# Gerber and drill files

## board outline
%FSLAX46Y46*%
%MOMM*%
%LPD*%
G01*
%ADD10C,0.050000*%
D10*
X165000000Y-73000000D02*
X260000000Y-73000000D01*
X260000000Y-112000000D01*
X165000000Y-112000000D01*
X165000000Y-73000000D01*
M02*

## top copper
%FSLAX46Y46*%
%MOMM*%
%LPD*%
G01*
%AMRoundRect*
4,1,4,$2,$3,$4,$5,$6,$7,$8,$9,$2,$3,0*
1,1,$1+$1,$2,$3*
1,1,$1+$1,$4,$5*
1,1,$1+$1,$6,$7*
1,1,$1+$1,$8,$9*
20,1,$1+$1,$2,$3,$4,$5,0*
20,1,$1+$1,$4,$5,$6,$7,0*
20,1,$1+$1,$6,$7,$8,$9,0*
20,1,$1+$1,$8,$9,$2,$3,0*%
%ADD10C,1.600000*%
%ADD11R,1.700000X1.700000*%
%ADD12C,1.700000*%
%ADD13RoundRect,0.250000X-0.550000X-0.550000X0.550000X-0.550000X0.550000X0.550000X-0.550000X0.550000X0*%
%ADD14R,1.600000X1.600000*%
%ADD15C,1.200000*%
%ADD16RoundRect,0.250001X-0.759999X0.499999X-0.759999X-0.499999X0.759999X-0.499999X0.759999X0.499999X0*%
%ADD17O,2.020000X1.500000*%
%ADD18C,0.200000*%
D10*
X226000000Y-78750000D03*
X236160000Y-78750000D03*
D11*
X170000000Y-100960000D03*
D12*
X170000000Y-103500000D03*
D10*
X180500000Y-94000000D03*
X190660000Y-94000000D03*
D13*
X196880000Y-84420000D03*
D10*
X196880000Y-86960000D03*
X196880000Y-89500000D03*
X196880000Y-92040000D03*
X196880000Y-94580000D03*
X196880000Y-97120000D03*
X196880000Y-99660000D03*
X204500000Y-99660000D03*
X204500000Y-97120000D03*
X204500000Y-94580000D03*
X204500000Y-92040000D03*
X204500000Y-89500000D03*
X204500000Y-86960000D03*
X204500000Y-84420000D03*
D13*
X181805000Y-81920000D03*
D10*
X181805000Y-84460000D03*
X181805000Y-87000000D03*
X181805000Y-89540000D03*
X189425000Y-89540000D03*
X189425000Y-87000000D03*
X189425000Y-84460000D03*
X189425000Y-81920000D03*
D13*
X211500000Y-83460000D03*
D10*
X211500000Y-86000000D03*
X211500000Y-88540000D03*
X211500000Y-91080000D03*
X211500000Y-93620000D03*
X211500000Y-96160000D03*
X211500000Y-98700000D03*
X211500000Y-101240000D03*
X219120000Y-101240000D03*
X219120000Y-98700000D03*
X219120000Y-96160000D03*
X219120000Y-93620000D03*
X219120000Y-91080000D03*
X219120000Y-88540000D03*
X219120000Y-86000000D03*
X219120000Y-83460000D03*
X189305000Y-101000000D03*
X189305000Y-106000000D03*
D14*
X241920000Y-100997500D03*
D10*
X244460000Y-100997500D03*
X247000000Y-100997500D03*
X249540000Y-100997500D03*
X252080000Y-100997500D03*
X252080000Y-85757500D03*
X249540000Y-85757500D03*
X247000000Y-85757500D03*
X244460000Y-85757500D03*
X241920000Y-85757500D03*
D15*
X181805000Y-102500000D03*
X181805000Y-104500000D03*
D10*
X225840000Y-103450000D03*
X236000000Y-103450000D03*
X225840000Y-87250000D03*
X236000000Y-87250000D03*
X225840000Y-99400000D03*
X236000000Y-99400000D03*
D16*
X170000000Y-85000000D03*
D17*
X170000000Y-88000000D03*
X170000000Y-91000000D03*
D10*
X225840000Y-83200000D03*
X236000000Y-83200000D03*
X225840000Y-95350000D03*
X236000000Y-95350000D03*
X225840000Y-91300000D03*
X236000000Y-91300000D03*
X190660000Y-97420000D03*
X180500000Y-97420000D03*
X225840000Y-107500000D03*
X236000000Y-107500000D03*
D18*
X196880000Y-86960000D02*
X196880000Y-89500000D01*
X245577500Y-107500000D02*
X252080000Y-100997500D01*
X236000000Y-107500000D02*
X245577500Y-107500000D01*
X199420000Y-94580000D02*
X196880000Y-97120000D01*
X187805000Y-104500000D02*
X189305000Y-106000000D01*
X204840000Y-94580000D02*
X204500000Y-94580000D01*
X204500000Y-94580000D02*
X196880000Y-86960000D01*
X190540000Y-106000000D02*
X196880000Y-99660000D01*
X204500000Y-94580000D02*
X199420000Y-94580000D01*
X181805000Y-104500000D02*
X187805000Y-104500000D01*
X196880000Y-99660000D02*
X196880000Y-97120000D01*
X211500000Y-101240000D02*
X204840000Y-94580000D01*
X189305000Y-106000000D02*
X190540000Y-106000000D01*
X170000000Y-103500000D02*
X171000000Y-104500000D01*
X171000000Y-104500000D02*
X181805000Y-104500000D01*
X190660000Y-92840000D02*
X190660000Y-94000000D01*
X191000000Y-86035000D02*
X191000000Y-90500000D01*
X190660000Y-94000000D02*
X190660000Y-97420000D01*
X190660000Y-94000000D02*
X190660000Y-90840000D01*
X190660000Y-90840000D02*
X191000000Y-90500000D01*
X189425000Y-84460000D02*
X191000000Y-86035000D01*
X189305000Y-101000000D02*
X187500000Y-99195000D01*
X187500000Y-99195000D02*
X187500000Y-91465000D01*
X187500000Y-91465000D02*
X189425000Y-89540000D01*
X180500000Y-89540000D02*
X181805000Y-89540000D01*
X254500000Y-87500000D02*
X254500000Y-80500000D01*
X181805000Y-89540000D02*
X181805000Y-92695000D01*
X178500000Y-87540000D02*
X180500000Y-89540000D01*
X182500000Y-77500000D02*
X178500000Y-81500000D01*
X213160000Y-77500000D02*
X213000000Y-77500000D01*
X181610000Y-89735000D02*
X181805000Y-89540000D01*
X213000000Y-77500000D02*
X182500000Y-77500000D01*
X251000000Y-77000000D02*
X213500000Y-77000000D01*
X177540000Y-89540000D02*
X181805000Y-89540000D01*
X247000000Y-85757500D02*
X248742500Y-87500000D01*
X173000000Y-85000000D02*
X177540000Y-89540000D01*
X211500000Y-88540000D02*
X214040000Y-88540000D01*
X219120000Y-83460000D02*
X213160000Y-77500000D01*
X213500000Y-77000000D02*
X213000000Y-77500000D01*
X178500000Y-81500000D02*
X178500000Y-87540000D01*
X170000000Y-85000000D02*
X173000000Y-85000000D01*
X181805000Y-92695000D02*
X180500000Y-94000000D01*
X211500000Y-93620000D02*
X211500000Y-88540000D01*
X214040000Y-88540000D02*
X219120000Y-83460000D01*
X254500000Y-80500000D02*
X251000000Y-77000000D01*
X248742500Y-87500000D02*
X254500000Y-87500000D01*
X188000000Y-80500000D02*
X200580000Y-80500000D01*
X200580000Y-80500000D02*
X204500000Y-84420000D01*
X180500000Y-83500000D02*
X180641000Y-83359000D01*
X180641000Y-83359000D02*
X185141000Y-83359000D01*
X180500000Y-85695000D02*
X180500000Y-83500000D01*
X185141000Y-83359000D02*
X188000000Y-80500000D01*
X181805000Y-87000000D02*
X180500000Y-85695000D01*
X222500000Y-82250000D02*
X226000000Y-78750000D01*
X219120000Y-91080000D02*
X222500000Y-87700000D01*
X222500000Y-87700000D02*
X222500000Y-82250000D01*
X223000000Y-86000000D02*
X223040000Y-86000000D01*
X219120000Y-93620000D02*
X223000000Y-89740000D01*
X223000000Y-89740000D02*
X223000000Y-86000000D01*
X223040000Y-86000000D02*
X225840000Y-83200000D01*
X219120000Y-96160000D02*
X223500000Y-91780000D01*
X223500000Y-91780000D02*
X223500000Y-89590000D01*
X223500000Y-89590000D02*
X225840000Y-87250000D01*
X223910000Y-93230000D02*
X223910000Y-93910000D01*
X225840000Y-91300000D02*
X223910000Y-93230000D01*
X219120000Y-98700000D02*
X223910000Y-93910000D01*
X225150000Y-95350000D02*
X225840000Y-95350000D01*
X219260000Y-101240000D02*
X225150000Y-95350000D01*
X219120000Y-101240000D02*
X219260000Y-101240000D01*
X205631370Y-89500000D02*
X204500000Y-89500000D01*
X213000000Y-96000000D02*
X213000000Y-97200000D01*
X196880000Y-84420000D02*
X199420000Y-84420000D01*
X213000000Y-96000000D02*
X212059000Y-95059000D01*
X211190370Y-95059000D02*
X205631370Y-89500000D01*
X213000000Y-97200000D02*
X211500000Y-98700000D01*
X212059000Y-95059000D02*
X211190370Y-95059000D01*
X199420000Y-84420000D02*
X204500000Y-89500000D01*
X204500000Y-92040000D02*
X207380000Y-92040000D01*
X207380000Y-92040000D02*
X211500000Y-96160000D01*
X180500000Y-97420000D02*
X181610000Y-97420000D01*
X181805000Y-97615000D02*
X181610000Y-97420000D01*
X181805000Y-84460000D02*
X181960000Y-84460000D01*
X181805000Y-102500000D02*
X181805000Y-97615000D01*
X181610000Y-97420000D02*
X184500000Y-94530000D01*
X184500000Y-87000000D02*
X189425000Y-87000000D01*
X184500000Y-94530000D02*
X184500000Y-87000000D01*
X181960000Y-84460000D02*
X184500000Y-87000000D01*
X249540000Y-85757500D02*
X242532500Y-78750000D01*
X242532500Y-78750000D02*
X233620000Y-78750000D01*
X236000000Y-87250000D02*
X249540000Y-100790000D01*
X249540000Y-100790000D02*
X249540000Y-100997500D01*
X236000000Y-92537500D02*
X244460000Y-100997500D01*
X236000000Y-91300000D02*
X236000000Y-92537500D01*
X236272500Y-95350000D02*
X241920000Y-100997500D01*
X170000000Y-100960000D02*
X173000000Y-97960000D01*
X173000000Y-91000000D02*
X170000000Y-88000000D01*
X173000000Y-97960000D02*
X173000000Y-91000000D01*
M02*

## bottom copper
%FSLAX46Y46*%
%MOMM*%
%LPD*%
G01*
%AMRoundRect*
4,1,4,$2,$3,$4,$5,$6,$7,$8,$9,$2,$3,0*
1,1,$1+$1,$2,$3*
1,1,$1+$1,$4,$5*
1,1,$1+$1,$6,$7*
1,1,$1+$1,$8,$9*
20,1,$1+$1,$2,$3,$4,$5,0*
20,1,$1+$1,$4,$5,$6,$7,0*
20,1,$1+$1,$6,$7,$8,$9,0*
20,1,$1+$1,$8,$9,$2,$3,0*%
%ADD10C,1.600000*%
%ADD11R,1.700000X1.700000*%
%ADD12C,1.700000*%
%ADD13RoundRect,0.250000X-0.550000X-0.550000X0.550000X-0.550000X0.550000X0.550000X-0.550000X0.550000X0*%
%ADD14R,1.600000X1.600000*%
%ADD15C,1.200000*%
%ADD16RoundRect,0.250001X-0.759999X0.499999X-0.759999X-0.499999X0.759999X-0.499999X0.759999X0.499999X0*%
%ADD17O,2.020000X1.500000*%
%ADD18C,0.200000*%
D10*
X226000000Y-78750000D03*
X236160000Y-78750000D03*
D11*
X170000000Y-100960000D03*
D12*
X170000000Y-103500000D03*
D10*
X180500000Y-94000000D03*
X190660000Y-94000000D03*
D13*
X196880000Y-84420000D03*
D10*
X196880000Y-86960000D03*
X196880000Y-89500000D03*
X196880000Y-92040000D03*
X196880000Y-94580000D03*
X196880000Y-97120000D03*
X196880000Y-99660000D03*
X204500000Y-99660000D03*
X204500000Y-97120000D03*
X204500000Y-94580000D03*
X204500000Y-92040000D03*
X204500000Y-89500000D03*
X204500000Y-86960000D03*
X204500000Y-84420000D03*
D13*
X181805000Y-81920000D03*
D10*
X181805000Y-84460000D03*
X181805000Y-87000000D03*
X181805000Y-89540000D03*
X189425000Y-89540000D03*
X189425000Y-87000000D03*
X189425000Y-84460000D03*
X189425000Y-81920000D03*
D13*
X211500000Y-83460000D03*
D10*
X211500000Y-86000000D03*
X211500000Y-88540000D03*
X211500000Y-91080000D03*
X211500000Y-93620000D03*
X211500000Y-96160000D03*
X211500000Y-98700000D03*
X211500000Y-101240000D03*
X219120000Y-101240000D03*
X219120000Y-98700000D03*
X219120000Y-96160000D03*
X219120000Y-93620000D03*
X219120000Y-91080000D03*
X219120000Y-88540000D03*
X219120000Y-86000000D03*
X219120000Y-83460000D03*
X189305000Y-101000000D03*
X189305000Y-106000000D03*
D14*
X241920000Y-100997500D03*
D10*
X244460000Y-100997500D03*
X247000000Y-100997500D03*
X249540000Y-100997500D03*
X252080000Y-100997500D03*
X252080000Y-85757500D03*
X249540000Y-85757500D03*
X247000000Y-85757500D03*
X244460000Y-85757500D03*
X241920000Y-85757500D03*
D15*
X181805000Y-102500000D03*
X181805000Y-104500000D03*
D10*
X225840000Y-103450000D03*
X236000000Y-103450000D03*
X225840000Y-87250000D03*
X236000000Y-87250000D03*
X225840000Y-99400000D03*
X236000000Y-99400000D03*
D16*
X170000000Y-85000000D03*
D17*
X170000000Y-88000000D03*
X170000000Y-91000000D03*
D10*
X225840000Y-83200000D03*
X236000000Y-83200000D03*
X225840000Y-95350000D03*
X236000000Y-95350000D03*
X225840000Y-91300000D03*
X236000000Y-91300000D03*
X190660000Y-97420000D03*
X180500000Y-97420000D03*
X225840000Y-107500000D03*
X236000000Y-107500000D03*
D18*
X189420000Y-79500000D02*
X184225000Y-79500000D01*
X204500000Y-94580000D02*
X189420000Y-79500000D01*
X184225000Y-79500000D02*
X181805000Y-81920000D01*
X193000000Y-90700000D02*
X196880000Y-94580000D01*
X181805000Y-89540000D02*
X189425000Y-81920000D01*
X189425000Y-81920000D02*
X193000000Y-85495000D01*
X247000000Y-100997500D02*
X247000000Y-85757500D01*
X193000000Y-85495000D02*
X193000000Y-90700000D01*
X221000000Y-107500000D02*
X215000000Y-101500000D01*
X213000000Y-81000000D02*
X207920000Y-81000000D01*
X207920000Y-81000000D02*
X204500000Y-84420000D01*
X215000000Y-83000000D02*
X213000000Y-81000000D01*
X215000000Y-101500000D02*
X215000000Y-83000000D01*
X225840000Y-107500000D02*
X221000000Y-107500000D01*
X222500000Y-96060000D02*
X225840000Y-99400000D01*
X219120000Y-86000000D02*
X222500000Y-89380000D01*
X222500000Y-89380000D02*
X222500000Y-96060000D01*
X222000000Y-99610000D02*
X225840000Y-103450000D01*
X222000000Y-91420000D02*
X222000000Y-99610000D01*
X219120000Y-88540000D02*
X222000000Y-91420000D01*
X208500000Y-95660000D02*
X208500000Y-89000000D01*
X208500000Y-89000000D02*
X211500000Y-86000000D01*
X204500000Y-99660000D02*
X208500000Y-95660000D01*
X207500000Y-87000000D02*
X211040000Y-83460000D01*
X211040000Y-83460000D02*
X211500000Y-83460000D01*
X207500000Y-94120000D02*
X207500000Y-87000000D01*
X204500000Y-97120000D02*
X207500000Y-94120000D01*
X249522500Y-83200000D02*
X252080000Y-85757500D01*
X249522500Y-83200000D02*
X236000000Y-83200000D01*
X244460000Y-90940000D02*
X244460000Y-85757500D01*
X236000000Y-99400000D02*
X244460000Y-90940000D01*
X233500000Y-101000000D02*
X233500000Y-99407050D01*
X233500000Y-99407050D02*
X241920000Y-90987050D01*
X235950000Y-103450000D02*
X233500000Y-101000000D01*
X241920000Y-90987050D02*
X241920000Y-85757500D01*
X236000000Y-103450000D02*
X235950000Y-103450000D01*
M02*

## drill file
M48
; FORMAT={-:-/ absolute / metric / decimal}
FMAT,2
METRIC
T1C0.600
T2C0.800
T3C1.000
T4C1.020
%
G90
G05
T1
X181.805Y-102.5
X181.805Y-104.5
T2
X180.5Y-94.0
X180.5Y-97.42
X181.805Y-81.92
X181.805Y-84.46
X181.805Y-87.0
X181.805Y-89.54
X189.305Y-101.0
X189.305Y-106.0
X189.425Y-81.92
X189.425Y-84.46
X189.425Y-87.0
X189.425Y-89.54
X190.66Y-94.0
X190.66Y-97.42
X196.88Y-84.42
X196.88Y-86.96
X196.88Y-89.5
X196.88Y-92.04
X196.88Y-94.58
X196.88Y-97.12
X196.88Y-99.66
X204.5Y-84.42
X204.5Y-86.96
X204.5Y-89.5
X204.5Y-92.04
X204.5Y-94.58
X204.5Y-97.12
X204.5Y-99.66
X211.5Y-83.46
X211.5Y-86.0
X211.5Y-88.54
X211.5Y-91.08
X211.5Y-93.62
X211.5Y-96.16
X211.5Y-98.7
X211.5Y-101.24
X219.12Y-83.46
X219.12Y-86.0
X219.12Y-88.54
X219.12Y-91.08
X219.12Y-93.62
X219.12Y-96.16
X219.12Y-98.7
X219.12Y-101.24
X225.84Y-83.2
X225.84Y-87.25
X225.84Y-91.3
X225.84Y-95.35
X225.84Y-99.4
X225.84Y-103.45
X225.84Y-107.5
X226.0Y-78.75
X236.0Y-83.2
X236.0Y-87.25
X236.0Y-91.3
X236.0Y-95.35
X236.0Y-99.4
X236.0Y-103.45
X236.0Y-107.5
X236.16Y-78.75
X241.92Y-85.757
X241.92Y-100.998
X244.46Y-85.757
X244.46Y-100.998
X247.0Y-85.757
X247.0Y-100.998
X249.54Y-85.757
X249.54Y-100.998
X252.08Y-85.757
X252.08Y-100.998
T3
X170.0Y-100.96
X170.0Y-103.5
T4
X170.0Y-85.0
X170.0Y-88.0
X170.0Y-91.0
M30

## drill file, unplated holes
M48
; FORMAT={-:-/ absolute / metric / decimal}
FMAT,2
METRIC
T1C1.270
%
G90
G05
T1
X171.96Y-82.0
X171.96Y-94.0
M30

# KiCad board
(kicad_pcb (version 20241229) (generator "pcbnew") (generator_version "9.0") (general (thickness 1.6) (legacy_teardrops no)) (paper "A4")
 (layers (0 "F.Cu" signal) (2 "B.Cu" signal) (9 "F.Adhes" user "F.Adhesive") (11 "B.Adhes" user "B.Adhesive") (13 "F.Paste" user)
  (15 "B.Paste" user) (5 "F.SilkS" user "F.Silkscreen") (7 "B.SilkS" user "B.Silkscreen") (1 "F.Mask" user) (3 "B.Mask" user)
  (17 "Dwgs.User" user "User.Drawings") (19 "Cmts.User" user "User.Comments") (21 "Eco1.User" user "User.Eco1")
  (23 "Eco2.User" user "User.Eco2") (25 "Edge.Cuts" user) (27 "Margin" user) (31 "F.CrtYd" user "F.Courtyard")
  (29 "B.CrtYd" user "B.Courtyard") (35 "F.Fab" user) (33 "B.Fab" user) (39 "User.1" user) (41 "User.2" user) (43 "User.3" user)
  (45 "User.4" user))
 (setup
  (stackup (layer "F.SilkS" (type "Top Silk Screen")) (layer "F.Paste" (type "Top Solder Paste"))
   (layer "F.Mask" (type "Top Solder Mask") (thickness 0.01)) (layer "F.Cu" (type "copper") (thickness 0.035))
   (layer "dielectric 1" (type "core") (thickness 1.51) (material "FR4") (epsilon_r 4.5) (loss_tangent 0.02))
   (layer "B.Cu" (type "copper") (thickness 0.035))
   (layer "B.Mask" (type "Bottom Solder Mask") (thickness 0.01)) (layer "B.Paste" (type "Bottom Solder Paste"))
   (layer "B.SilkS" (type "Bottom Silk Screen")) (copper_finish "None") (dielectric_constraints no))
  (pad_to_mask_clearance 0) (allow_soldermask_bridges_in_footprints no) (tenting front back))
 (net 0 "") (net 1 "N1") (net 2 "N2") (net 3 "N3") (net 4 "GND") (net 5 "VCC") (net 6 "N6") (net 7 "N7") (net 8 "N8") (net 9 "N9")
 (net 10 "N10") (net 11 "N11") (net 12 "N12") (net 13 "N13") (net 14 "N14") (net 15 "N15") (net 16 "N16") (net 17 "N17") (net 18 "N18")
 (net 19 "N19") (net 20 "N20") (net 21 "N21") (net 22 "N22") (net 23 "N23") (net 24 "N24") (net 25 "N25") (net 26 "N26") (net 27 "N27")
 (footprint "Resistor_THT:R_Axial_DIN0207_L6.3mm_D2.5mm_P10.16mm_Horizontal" (layer "F.Cu") (at 226 78.75)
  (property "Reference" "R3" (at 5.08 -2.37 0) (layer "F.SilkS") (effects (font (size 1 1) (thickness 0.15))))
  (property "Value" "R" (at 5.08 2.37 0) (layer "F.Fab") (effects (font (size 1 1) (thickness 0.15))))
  (pad "1" thru_hole circle (at 0 0) (size 1.6 1.6) (drill 0.8) (layers "*.Cu" "*.Mask") (remove_unused_layers no) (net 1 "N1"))
  (pad "2" thru_hole circle (at 10.16 0) (size 1.6 1.6) (drill 0.8) (layers "*.Cu" "*.Mask") (remove_unused_layers no) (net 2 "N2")))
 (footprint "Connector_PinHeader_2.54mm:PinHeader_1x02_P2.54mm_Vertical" (layer "F.Cu") (at 170 100.96)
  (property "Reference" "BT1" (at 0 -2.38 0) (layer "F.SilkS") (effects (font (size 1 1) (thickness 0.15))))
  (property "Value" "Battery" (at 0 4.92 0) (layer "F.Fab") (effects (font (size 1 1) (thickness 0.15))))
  (pad "1" thru_hole rect (at 0 0) (size 1.7 1.7) (drill 1) (layers "*.Cu" "*.Mask") (remove_unused_layers no) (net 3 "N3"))
  (pad "2" thru_hole circle (at 0 2.54) (size 1.7 1.7) (drill 1) (layers "*.Cu" "*.Mask") (remove_unused_layers no) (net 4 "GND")))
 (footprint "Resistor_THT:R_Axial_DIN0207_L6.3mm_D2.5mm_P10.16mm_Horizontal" (layer "F.Cu") (at 180.5 94)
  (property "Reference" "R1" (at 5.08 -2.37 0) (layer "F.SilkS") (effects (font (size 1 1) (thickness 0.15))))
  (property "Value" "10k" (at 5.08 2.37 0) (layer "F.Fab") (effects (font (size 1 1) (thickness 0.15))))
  (pad "1" thru_hole circle (at 0 0) (size 1.6 1.6) (drill 0.8) (layers "*.Cu" "*.Mask") (remove_unused_layers no) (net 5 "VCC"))
  (pad "2" thru_hole circle (at 10.16 0) (size 1.6 1.6) (drill 0.8) (layers "*.Cu" "*.Mask") (remove_unused_layers no) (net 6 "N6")))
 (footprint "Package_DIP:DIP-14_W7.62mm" (layer "F.Cu") (at 196.88 84.42)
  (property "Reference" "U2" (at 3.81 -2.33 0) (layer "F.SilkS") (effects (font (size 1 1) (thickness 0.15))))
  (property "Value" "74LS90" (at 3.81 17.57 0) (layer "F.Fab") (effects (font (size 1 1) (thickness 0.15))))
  (pad "1" thru_hole roundrect (at 0 0) (size 1.6 1.6) (drill 0.8) (layers "*.Cu" "*.Mask") (remove_unused_layers no)
   (roundrect_rratio 0.15625) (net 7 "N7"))
  (pad "2" thru_hole circle (at 0 2.54) (size 1.6 1.6) (drill 0.8) (layers "*.Cu" "*.Mask") (remove_unused_layers no) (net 4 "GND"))
  (pad "3" thru_hole circle (at 0 5.08) (size 1.6 1.6) (drill 0.8) (layers "*.Cu" "*.Mask") (remove_unused_layers no) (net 4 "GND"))
  (pad "4" thru_hole circle (at 0 7.62) (size 1.6 1.6) (drill 0.8) (layers "*.Cu" "*.Mask") (remove_unused_layers no))
  (pad "5" thru_hole circle (at 0 10.16) (size 1.6 1.6) (drill 0.8) (layers "*.Cu" "*.Mask") (remove_unused_layers no) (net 5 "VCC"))
  (pad "6" thru_hole circle (at 0 12.7) (size 1.6 1.6) (drill 0.8) (layers "*.Cu" "*.Mask") (remove_unused_layers no) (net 4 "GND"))
  (pad "7" thru_hole circle (at 0 15.24) (size 1.6 1.6) (drill 0.8) (layers "*.Cu" "*.Mask") (remove_unused_layers no) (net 4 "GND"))
  (pad "8" thru_hole circle (at 7.62 15.24) (size 1.6 1.6) (drill 0.8) (layers "*.Cu" "*.Mask") (remove_unused_layers no) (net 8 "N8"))
  (pad "9" thru_hole circle (at 7.62 12.7) (size 1.6 1.6) (drill 0.8) (layers "*.Cu" "*.Mask") (remove_unused_layers no) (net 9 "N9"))
  (pad "10" thru_hole circle (at 7.62 10.16) (size 1.6 1.6) (drill 0.8) (layers "*.Cu" "*.Mask") (remove_unused_layers no) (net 4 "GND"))
  (pad "11" thru_hole circle (at 7.62 7.62) (size 1.6 1.6) (drill 0.8) (layers "*.Cu" "*.Mask") (remove_unused_layers no) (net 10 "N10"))
  (pad "12" thru_hole circle (at 7.62 5.08) (size 1.6 1.6) (drill 0.8) (layers "*.Cu" "*.Mask") (remove_unused_layers no) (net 7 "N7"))
  (pad "13" thru_hole circle (at 7.62 2.54) (size 1.6 1.6) (drill 0.8) (layers "*.Cu" "*.Mask") (remove_unused_layers no))
  (pad "14" thru_hole circle (at 7.62 0) (size 1.6 1.6) (drill 0.8) (layers "*.Cu" "*.Mask") (remove_unused_layers no) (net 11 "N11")))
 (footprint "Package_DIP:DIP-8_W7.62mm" (layer "F.Cu") (at 181.805 81.92)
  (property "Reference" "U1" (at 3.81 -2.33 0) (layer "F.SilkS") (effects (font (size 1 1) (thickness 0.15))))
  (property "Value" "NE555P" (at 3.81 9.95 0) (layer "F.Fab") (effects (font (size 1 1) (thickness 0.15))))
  (pad "1" thru_hole roundrect (at 0 0) (size 1.6 1.6) (drill 0.8) (layers "*.Cu" "*.Mask") (remove_unused_layers no)
   (roundrect_rratio 0.15625) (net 4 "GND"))
  (pad "2" thru_hole circle (at 0 2.54) (size 1.6 1.6) (drill 0.8) (layers "*.Cu" "*.Mask") (remove_unused_layers no) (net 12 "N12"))
  (pad "3" thru_hole circle (at 0 5.08) (size 1.6 1.6) (drill 0.8) (layers "*.Cu" "*.Mask") (remove_unused_layers no) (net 11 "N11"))
  (pad "4" thru_hole circle (at 0 7.62) (size 1.6 1.6) (drill 0.8) (layers "*.Cu" "*.Mask") (remove_unused_layers no) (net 5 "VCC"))
  (pad "5" thru_hole circle (at 7.62 7.62) (size 1.6 1.6) (drill 0.8) (layers "*.Cu" "*.Mask") (remove_unused_layers no) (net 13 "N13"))
  (pad "6" thru_hole circle (at 7.62 5.08) (size 1.6 1.6) (drill 0.8) (layers "*.Cu" "*.Mask") (remove_unused_layers no) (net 12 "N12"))
  (pad "7" thru_hole circle (at 7.62 2.54) (size 1.6 1.6) (drill 0.8) (layers "*.Cu" "*.Mask") (remove_unused_layers no) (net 6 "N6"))
  (pad "8" thru_hole circle (at 7.62 0) (size 1.6 1.6) (drill 0.8) (layers "*.Cu" "*.Mask") (remove_unused_layers no) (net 5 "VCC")))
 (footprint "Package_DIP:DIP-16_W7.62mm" (layer "F.Cu") (at 211.5 83.46)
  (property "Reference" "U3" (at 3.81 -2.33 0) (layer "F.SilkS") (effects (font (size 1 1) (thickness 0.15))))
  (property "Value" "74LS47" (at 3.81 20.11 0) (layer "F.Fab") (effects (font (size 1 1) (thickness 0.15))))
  (pad "1" thru_hole roundrect (at 0 0) (size 1.6 1.6) (drill 0.8) (layers "*.Cu" "*.Mask") (remove_unused_layers no)
   (roundrect_rratio 0.15625) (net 9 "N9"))
  (pad "2" thru_hole circle (at 0 2.54) (size 1.6 1.6) (drill 0.8) (layers "*.Cu" "*.Mask") (remove_unused_layers no) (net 8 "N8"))
  (pad "3" thru_hole circle (at 0 5.08) (size 1.6 1.6) (drill 0.8) (layers "*.Cu" "*.Mask") (remove_unused_layers no) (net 5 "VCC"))
  (pad "4" thru_hole circle (at 0 7.62) (size 1.6 1.6) (drill 0.8) (layers "*.Cu" "*.Mask") (remove_unused_layers no) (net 5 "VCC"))
  (pad "5" thru_hole circle (at 0 10.16) (size 1.6 1.6) (drill 0.8) (layers "*.Cu" "*.Mask") (remove_unused_layers no) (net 5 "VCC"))
  (pad "6" thru_hole circle (at 0 12.7) (size 1.6 1.6) (drill 0.8) (layers "*.Cu" "*.Mask") (remove_unused_layers no) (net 10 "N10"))
  (pad "7" thru_hole circle (at 0 15.24) (size 1.6 1.6) (drill 0.8) (layers "*.Cu" "*.Mask") (remove_unused_layers no) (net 7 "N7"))
  (pad "8" thru_hole circle (at 0 17.78) (size 1.6 1.6) (drill 0.8) (layers "*.Cu" "*.Mask") (remove_unused_layers no) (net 4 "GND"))
  (pad "9" thru_hole circle (at 7.62 17.78) (size 1.6 1.6) (drill 0.8) (layers "*.Cu" "*.Mask") (remove_unused_layers no) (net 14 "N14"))
  (pad "10" thru_hole circle (at 7.62 15.24) (size 1.6 1.6) (drill 0.8) (layers "*.Cu" "*.Mask") (remove_unused_layers no) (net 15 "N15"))
  (pad "11" thru_hole circle (at 7.62 12.7) (size 1.6 1.6) (drill 0.8) (layers "*.Cu" "*.Mask") (remove_unused_layers no) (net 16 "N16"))
  (pad "12" thru_hole circle (at 7.62 10.16) (size 1.6 1.6) (drill 0.8) (layers "*.Cu" "*.Mask") (remove_unused_layers no) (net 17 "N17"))
  (pad "13" thru_hole circle (at 7.62 7.62) (size 1.6 1.6) (drill 0.8) (layers "*.Cu" "*.Mask") (remove_unused_layers no) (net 1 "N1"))
  (pad "14" thru_hole circle (at 7.62 5.08) (size 1.6 1.6) (drill 0.8) (layers "*.Cu" "*.Mask") (remove_unused_layers no) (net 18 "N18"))
  (pad "15" thru_hole circle (at 7.62 2.54) (size 1.6 1.6) (drill 0.8) (layers "*.Cu" "*.Mask") (remove_unused_layers no) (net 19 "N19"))
  (pad "16" thru_hole circle (at 7.62 0) (size 1.6 1.6) (drill 0.8) (layers "*.Cu" "*.Mask") (remove_unused_layers no) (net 5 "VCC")))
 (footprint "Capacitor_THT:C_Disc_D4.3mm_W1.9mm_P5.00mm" (layer "F.Cu") (at 189.305 101 -90)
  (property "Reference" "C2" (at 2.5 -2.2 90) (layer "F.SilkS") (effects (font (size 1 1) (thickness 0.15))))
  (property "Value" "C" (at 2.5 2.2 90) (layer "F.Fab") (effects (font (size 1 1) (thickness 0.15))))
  (pad "1" thru_hole circle (at 0 0 270) (size 1.6 1.6) (drill 0.8) (layers "*.Cu" "*.Mask") (remove_unused_layers no) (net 13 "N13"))
  (pad "2" thru_hole circle (at 5 0 270) (size 1.6 1.6) (drill 0.8) (layers "*.Cu" "*.Mask") (remove_unused_layers no) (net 4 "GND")))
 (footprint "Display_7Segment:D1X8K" (layer "F.Cu") (at 241.92 100.9975 90)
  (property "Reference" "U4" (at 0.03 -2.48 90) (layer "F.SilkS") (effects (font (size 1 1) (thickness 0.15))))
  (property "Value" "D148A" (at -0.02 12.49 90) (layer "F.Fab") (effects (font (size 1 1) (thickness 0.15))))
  (pad "1" thru_hole rect (at 0 0) (size 1.6 1.6) (drill 0.8) (layers "*.Cu" "*.Mask") (remove_unused_layers no) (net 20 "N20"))
  (pad "2" thru_hole circle (at 0 2.54) (size 1.6 1.6) (drill 0.8) (layers "*.Cu" "*.Mask") (remove_unused_layers no) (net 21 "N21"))
  (pad "3" thru_hole circle (at 0 5.08) (size 1.6 1.6) (drill 0.8) (layers "*.Cu" "*.Mask") (remove_unused_layers no) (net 5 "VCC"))
  (pad "4" thru_hole circle (at 0 7.62) (size 1.6 1.6) (drill 0.8) (layers "*.Cu" "*.Mask") (remove_unused_layers no) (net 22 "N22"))
  (pad "5" thru_hole circle (at 0 10.16) (size 1.6 1.6) (drill 0.8) (layers "*.Cu" "*.Mask") (remove_unused_layers no) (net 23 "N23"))
  (pad "6" thru_hole circle (at 15.24 10.16) (size 1.6 1.6) (drill 0.8) (layers "*.Cu" "*.Mask") (remove_unused_layers no) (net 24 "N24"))
  (pad "7" thru_hole circle (at 15.24 7.62) (size 1.6 1.6) (drill 0.8) (layers "*.Cu" "*.Mask") (remove_unused_layers no) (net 2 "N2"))
  (pad "8" thru_hole circle (at 15.24 5.08) (size 1.6 1.6) (drill 0.8) (layers "*.Cu" "*.Mask") (remove_unused_layers no) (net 5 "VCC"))
  (pad "9" thru_hole circle (at 15.24 2.54) (size 1.6 1.6) (drill 0.8) (layers "*.Cu" "*.Mask") (remove_unused_layers no) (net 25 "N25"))
  (pad "10" thru_hole circle (at 15.24 0) (size 1.6 1.6) (drill 0.8) (layers "*.Cu" "*.Mask") (remove_unused_layers no) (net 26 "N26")))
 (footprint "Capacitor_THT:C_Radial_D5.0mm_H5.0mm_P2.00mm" (layer "F.Cu") (at 181.805 102.5 -90)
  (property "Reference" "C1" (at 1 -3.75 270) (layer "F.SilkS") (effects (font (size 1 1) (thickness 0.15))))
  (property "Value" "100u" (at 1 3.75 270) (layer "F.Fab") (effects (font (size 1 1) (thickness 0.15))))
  (pad "1" thru_hole circle (at 0 0 270) (size 1.2 1.2) (drill 0.6) (layers "*.Cu" "*.Mask") (remove_unused_layers no) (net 12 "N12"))
  (pad "2" thru_hole circle (at 2 0 270) (size 1.2 1.2) (drill 0.6) (layers "*.Cu" "*.Mask") (remove_unused_layers no) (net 4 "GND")))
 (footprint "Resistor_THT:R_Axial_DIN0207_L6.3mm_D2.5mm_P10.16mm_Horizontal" (layer "F.Cu") (at 225.84 103.45)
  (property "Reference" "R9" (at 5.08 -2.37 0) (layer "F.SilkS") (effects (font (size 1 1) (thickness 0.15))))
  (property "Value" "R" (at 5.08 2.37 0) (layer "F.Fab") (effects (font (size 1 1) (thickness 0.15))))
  (pad "1" thru_hole circle (at 0 0) (size 1.6 1.6) (drill 0.8) (layers "*.Cu" "*.Mask") (remove_unused_layers no) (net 18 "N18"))
  (pad "2" thru_hole circle (at 10.16 0) (size 1.6 1.6) (drill 0.8) (layers "*.Cu" "*.Mask") (remove_unused_layers no) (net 26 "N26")))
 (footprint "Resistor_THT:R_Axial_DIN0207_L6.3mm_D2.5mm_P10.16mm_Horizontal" (layer "F.Cu") (at 225.84 87.25)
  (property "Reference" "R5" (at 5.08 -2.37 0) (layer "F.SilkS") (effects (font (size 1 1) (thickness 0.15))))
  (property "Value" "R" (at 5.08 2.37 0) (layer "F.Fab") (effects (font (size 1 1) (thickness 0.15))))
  (pad "1" thru_hole circle (at 0 0) (size 1.6 1.6) (drill 0.8) (layers "*.Cu" "*.Mask") (remove_unused_layers no) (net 16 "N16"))
  (pad "2" thru_hole circle (at 10.16 0) (size 1.6 1.6) (drill 0.8) (layers "*.Cu" "*.Mask") (remove_unused_layers no) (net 22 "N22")))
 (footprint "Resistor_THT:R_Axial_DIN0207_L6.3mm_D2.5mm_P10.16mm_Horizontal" (layer "F.Cu") (at 225.84 99.4)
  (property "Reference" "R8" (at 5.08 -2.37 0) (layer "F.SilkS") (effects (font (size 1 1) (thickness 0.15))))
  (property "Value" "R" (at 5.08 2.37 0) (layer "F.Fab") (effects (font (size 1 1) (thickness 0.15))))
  (pad "1" thru_hole circle (at 0 0) (size 1.6 1.6) (drill 0.8) (layers "*.Cu" "*.Mask") (remove_unused_layers no) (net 19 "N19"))
  (pad "2" thru_hole circle (at 10.16 0) (size 1.6 1.6) (drill 0.8) (layers "*.Cu" "*.Mask") (remove_unused_layers no) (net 25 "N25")))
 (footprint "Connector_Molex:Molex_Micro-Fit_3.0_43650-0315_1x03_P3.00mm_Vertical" (layer "F.Cu") (at 170 85 -90)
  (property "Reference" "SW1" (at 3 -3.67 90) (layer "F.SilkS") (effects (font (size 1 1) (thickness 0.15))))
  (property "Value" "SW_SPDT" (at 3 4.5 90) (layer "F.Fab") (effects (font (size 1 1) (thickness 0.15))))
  (pad "" np_thru_hole circle (at -3 -1.96 270) (size 1.27 1.27) (drill 1.27) (layers "*.Cu" "*.Mask"))
  (pad "" np_thru_hole circle (at 9 -1.96 270) (size 1.27 1.27) (drill 1.27) (layers "*.Cu" "*.Mask"))
  (pad "1" thru_hole roundrect (at 0 0 270) (size 1.5 2.02) (drill 1.02) (layers "*.Cu" "*.Mask") (remove_unused_layers no)
   (roundrect_rratio 0.166667) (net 5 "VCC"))
  (pad "2" thru_hole oval (at 3 0 270) (size 1.5 2.02) (drill 1.02) (layers "*.Cu" "*.Mask") (remove_unused_layers no) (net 3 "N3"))
  (pad "3" thru_hole oval (at 6 0 270) (size 1.5 2.02) (drill 1.02) (layers "*.Cu" "*.Mask") (remove_unused_layers no) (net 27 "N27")))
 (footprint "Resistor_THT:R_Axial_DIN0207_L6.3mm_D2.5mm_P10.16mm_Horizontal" (layer "F.Cu") (at 225.84 83.2)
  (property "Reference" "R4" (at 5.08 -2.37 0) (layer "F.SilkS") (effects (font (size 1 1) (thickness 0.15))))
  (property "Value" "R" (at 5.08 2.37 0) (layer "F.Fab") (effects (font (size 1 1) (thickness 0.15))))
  (pad "1" thru_hole circle (at 0 0) (size 1.6 1.6) (drill 0.8) (layers "*.Cu" "*.Mask") (remove_unused_layers no) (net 17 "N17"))
  (pad "2" thru_hole circle (at 10.16 0) (size 1.6 1.6) (drill 0.8) (layers "*.Cu" "*.Mask") (remove_unused_layers no) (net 24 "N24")))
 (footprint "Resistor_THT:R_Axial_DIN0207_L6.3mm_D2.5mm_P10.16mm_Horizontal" (layer "F.Cu") (at 225.84 95.35)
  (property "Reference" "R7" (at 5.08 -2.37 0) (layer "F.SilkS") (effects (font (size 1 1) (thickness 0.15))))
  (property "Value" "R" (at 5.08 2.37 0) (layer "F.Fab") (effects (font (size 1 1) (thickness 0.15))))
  (pad "1" thru_hole circle (at 0 0) (size 1.6 1.6) (drill 0.8) (layers "*.Cu" "*.Mask") (remove_unused_layers no) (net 14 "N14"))
  (pad "2" thru_hole circle (at 10.16 0) (size 1.6 1.6) (drill 0.8) (layers "*.Cu" "*.Mask") (remove_unused_layers no) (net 20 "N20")))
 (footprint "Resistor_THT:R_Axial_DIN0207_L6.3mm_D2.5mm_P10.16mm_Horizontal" (layer "F.Cu") (at 225.84 91.3)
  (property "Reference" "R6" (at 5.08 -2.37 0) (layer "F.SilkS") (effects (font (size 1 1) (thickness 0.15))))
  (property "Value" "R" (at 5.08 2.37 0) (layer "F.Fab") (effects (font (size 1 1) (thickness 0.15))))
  (pad "1" thru_hole circle (at 0 0) (size 1.6 1.6) (drill 0.8) (layers "*.Cu" "*.Mask") (remove_unused_layers no) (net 15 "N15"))
  (pad "2" thru_hole circle (at 10.16 0) (size 1.6 1.6) (drill 0.8) (layers "*.Cu" "*.Mask") (remove_unused_layers no) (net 21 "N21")))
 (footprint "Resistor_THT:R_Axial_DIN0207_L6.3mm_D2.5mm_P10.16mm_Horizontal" (layer "F.Cu") (at 190.66 97.42 180)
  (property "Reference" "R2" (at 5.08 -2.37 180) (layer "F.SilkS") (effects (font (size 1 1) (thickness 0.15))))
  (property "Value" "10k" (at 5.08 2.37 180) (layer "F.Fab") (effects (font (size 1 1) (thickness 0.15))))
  (pad "1" thru_hole circle (at 0 0 180) (size 1.6 1.6) (drill 0.8) (layers "*.Cu" "*.Mask") (remove_unused_layers no) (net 6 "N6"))
  (pad "2" thru_hole circle (at 10.16 0 180) (size 1.6 1.6) (drill 0.8) (layers "*.Cu" "*.Mask") (remove_unused_layers no) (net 12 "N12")))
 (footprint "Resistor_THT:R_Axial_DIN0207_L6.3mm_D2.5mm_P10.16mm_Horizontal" (layer "F.Cu") (at 225.84 107.5)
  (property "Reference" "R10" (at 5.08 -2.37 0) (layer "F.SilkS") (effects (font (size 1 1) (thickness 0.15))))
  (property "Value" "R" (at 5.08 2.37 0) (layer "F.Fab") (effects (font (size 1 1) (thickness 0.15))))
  (pad "1" thru_hole circle (at 0 0) (size 1.6 1.6) (drill 0.8) (layers "*.Cu" "*.Mask") (remove_unused_layers no) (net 11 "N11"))
  (pad "2" thru_hole circle (at 10.16 0) (size 1.6 1.6) (drill 0.8) (layers "*.Cu" "*.Mask") (remove_unused_layers no) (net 23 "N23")))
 (gr_rect (start 165 73) (end 260 112) (stroke (width 0.05) (type default)) (fill no) (layer "Edge.Cuts"))
 (segment (start 199.42 94.58) (end 196.88 97.12) (width 0.2) (layer "F.Cu") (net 4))
 (segment (start 187.805 104.5) (end 189.305 106) (width 0.2) (layer "F.Cu") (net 4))
 (segment (start 204.84 94.58) (end 204.5 94.58) (width 0.2) (layer "F.Cu") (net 4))
 (segment (start 196.88 86.96) (end 196.88 89.5) (width 0.2) (layer "F.Cu") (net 4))
 (segment (start 204.5 94.58) (end 196.88 86.96) (width 0.2) (layer "F.Cu") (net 4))
 (segment (start 190.54 106) (end 196.88 99.66) (width 0.2) (layer "F.Cu") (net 4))
 (segment (start 204.5 94.58) (end 199.42 94.58) (width 0.2) (layer "F.Cu") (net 4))
 (segment (start 181.805 104.5) (end 187.805 104.5) (width 0.2) (layer "F.Cu") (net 4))
 (segment (start 196.88 99.66) (end 196.88 97.12) (width 0.2) (layer "F.Cu") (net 4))
 (segment (start 211.5 101.24) (end 204.84 94.58) (width 0.2) (layer "F.Cu") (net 4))
 (segment (start 189.305 106) (end 190.54 106) (width 0.2) (layer "F.Cu") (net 4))
 (segment (start 170 103.5) (end 171 104.5) (width 0.2) (layer "F.Cu") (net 4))
 (segment (start 171 104.5) (end 181.805 104.5) (width 0.2) (layer "F.Cu") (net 4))
 (segment (start 189.42 79.5) (end 184.225 79.5) (width 0.2) (layer "B.Cu") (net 4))
 (segment (start 204.5 94.58) (end 189.42 79.5) (width 0.2) (layer "B.Cu") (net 4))
 (segment (start 184.225 79.5) (end 181.805 81.92) (width 0.2) (layer "B.Cu") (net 4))
 (segment (start 190.66 92.84) (end 190.66 94) (width 0.2) (layer "F.Cu") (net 6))
 (segment (start 191 86.035) (end 191 90.5) (width 0.2) (layer "F.Cu") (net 6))
 (segment (start 190.66 94) (end 190.66 97.42) (width 0.2) (layer "F.Cu") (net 6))
 (segment (start 190.66 94) (end 190.66 90.84) (width 0.2) (layer "F.Cu") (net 6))
 (segment (start 190.66 90.84) (end 191 90.5) (width 0.2) (layer "F.Cu") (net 6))
 (segment (start 189.425 84.46) (end 191 86.035) (width 0.2) (layer "F.Cu") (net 6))
 (segment (start 189.305 101) (end 187.5 99.195) (width 0.2) (layer "F.Cu") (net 13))
 (segment (start 187.5 99.195) (end 187.5 91.465) (width 0.2) (layer "F.Cu") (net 13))
 (segment (start 187.5 91.465) (end 189.425 89.54) (width 0.2) (layer "F.Cu") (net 13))
 (segment (start 180.5 89.54) (end 181.805 89.54) (width 0.2) (layer "F.Cu") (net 5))
 (segment (start 254.5 87.5) (end 254.5 80.5) (width 0.2) (layer "F.Cu") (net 5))
 (segment (start 181.805 89.54) (end 181.805 92.695) (width 0.2) (layer "F.Cu") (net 5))
 (segment (start 178.5 87.54) (end 180.5 89.54) (width 0.2) (layer "F.Cu") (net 5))
 (segment (start 182.5 77.5) (end 178.5 81.5) (width 0.2) (layer "F.Cu") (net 5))
 (segment (start 213.16 77.5) (end 213 77.5) (width 0.2) (layer "F.Cu") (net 5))
 (segment (start 181.61 89.735) (end 181.805 89.54) (width 0.2) (layer "F.Cu") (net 5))
 (segment (start 213 77.5) (end 182.5 77.5) (width 0.2) (layer "F.Cu") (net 5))
 (segment (start 251 77) (end 213.5 77) (width 0.2) (layer "F.Cu") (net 5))
 (segment (start 177.54 89.54) (end 181.805 89.54) (width 0.2) (layer "F.Cu") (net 5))
 (segment (start 247 85.7575) (end 248.7425 87.5) (width 0.2) (layer "F.Cu") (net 5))
 (segment (start 173 85) (end 177.54 89.54) (width 0.2) (layer "F.Cu") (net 5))
 (segment (start 211.5 88.54) (end 214.04 88.54) (width 0.2) (layer "F.Cu") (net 5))
 (segment (start 219.12 83.46) (end 213.16 77.5) (width 0.2) (layer "F.Cu") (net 5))
 (segment (start 213.5 77) (end 213 77.5) (width 0.2) (layer "F.Cu") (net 5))
 (segment (start 178.5 81.5) (end 178.5 87.54) (width 0.2) (layer "F.Cu") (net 5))
 (segment (start 170 85) (end 173 85) (width 0.2) (layer "F.Cu") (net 5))
 (segment (start 181.805 92.695) (end 180.5 94) (width 0.2) (layer "F.Cu") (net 5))
 (segment (start 211.5 93.62) (end 211.5 88.54) (width 0.2) (layer "F.Cu") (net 5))
 (segment (start 214.04 88.54) (end 219.12 83.46) (width 0.2) (layer "F.Cu") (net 5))
 (segment (start 254.5 80.5) (end 251 77) (width 0.2) (layer "F.Cu") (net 5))
 (segment (start 248.7425 87.5) (end 254.5 87.5) (width 0.2) (layer "F.Cu") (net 5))
 (segment (start 193 90.7) (end 196.88 94.58) (width 0.2) (layer "B.Cu") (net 5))
 (segment (start 181.805 89.54) (end 189.425 81.92) (width 0.2) (layer "B.Cu") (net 5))
 (segment (start 189.425 81.92) (end 193 85.495) (width 0.2) (layer "B.Cu") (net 5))
 (segment (start 247 100.9975) (end 247 85.7575) (width 0.2) (layer "B.Cu") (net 5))
 (segment (start 193 85.495) (end 193 90.7) (width 0.2) (layer "B.Cu") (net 5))
 (segment (start 188 80.5) (end 200.58 80.5) (width 0.2) (layer "F.Cu") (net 11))
 (segment (start 200.58 80.5) (end 204.5 84.42) (width 0.2) (layer "F.Cu") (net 11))
 (segment (start 180.5 83.5) (end 180.641 83.359) (width 0.2) (layer "F.Cu") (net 11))
 (segment (start 180.641 83.359) (end 185.141 83.359) (width 0.2) (layer "F.Cu") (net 11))
 (segment (start 180.5 85.695) (end 180.5 83.5) (width 0.2) (layer "F.Cu") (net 11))
 (segment (start 185.141 83.359) (end 188 80.5) (width 0.2) (layer "F.Cu") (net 11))
 (segment (start 181.805 87) (end 180.5 85.695) (width 0.2) (layer "F.Cu") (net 11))
 (segment (start 221 107.5) (end 215 101.5) (width 0.2) (layer "B.Cu") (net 11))
 (segment (start 213 81) (end 207.92 81) (width 0.2) (layer "B.Cu") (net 11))
 (segment (start 207.92 81) (end 204.5 84.42) (width 0.2) (layer "B.Cu") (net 11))
 (segment (start 215 83) (end 213 81) (width 0.2) (layer "B.Cu") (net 11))
 (segment (start 215 101.5) (end 215 83) (width 0.2) (layer "B.Cu") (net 11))
 (segment (start 225.84 107.5) (end 221 107.5) (width 0.2) (layer "B.Cu") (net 11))
 (segment (start 222.5 82.25) (end 226 78.75) (width 0.2) (layer "F.Cu") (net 1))
 (segment (start 219.12 91.08) (end 222.5 87.7) (width 0.2) (layer "F.Cu") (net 1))
 (segment (start 222.5 87.7) (end 222.5 82.25) (width 0.2) (layer "F.Cu") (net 1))
 (segment (start 223 86) (end 223.04 86) (width 0.2) (layer "F.Cu") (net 17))
 (segment (start 219.12 93.62) (end 223 89.74) (width 0.2) (layer "F.Cu") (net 17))
 (segment (start 223 89.74) (end 223 86) (width 0.2) (layer "F.Cu") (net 17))
 (segment (start 223.04 86) (end 225.84 83.2) (width 0.2) (layer "F.Cu") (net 17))
 (segment (start 219.12 96.16) (end 223.5 91.78) (width 0.2) (layer "F.Cu") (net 16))
 (segment (start 223.5 91.78) (end 223.5 89.59) (width 0.2) (layer "F.Cu") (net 16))
 (segment (start 223.5 89.59) (end 225.84 87.25) (width 0.2) (layer "F.Cu") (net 16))
 (segment (start 223.91 93.23) (end 223.91 93.91) (width 0.2) (layer "F.Cu") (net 15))
 (segment (start 225.84 91.3) (end 223.91 93.23) (width 0.2) (layer "F.Cu") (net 15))
 (segment (start 219.12 98.7) (end 223.91 93.91) (width 0.2) (layer "F.Cu") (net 15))
 (segment (start 225.15 95.35) (end 225.84 95.35) (width 0.2) (layer "F.Cu") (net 14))
 (segment (start 219.26 101.24) (end 225.15 95.35) (width 0.2) (layer "F.Cu") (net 14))
 (segment (start 219.12 101.24) (end 219.26 101.24) (width 0.2) (layer "F.Cu") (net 14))
 (segment (start 222.5 96.06) (end 225.84 99.4) (width 0.2) (layer "B.Cu") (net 19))
 (segment (start 219.12 86) (end 222.5 89.38) (width 0.2) (layer "B.Cu") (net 19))
 (segment (start 222.5 89.38) (end 222.5 96.06) (width 0.2) (layer "B.Cu") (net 19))
 (segment (start 222 99.61) (end 225.84 103.45) (width 0.2) (layer "B.Cu") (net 18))
 (segment (start 222 91.42) (end 222 99.61) (width 0.2) (layer "B.Cu") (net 18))
 (segment (start 219.12 88.54) (end 222 91.42) (width 0.2) (layer "B.Cu") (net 18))
 (segment (start 208.5 95.66) (end 208.5 89) (width 0.2) (layer "B.Cu") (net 8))
 (segment (start 208.5 89) (end 211.5 86) (width 0.2) (layer "B.Cu") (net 8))
 (segment (start 204.5 99.66) (end 208.5 95.66) (width 0.2) (layer "B.Cu") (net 8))
 (segment (start 205.63137 89.5) (end 204.5 89.5) (width 0.2) (layer "F.Cu") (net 7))
 (segment (start 213 96) (end 213 97.2) (width 0.2) (layer "F.Cu") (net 7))
 (segment (start 196.88 84.42) (end 199.42 84.42) (width 0.2) (layer "F.Cu") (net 7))
 (segment (start 213 96) (end 212.059 95.059) (width 0.2) (layer "F.Cu") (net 7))
 (segment (start 211.19037 95.059) (end 205.63137 89.5) (width 0.2) (layer "F.Cu") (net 7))
 (segment (start 213 97.2) (end 211.5 98.7) (width 0.2) (layer "F.Cu") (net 7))
 (segment (start 212.059 95.059) (end 211.19037 95.059) (width 0.2) (layer "F.Cu") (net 7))
 (segment (start 199.42 84.42) (end 204.5 89.5) (width 0.2) (layer "F.Cu") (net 7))
 (segment (start 204.5 92.04) (end 207.38 92.04) (width 0.2) (layer "F.Cu") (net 10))
 (segment (start 207.38 92.04) (end 211.5 96.16) (width 0.2) (layer "F.Cu") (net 10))
 (segment (start 207.5 87) (end 211.04 83.46) (width 0.2) (layer "B.Cu") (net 9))
 (segment (start 211.04 83.46) (end 211.5 83.46) (width 0.2) (layer "B.Cu") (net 9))
 (segment (start 207.5 94.12) (end 207.5 87) (width 0.2) (layer "B.Cu") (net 9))
 (segment (start 204.5 97.12) (end 207.5 94.12) (width 0.2) (layer "B.Cu") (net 9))
 (segment (start 180.5 97.42) (end 181.61 97.42) (width 0.2) (layer "F.Cu") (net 12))
 (segment (start 181.805 97.615) (end 181.61 97.42) (width 0.2) (layer "F.Cu") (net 12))
 (segment (start 181.805 84.46) (end 181.96 84.46) (width 0.2) (layer "F.Cu") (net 12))
 (segment (start 181.805 102.5) (end 181.805 97.615) (width 0.2) (layer "F.Cu") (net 12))
 (segment (start 181.61 97.42) (end 184.5 94.53) (width 0.2) (layer "F.Cu") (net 12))
 (segment (start 184.5 87) (end 189.425 87) (width 0.2) (layer "F.Cu") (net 12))
 (segment (start 184.5 94.53) (end 184.5 87) (width 0.2) (layer "F.Cu") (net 12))
 (segment (start 181.96 84.46) (end 184.5 87) (width 0.2) (layer "F.Cu") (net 12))
 (segment (start 249.54 85.7575) (end 242.5325 78.75) (width 0.2) (layer "F.Cu") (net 2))
 (segment (start 242.5325 78.75) (end 233.62 78.75) (width 0.2) (layer "F.Cu") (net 2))
 (segment (start 249.5225 83.2) (end 252.08 85.7575) (width 0.2) (layer "B.Cu") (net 24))
 (segment (start 249.5225 83.2) (end 236 83.2) (width 0.2) (layer "B.Cu") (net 24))
 (segment (start 236 87.25) (end 249.54 100.79) (width 0.2) (layer "F.Cu") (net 22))
 (segment (start 249.54 100.79) (end 249.54 100.9975) (width 0.2) (layer "F.Cu") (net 22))
 (segment (start 236 92.5375) (end 244.46 100.9975) (width 0.2) (layer "F.Cu") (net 21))
 (segment (start 236 91.3) (end 236 92.5375) (width 0.2) (layer "F.Cu") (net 21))
 (segment (start 236.2725 95.35) (end 241.92 100.9975) (width 0.2) (layer "F.Cu") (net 20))
 (segment (start 244.46 90.94) (end 244.46 85.7575) (width 0.2) (layer "B.Cu") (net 25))
 (segment (start 236 99.4) (end 244.46 90.94) (width 0.2) (layer "B.Cu") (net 25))
 (segment (start 233.5 101) (end 233.5 99.40705) (width 0.2) (layer "B.Cu") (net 26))
 (segment (start 233.5 99.40705) (end 241.92 90.98705) (width 0.2) (layer "B.Cu") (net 26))
 (segment (start 235.95 103.45) (end 233.5 101) (width 0.2) (layer "B.Cu") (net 26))
 (segment (start 241.92 90.98705) (end 241.92 85.7575) (width 0.2) (layer "B.Cu") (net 26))
 (segment (start 236 103.45) (end 235.95 103.45) (width 0.2) (layer "B.Cu") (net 26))
 (segment (start 236 107.5) (end 245.5775 107.5) (width 0.2) (layer "F.Cu") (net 23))
 (segment (start 245.5775 107.5) (end 252.08 100.9975) (width 0.2) (layer "F.Cu") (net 23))
 (segment (start 170 100.96) (end 173 97.96) (width 0.2) (layer "F.Cu") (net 3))
 (segment (start 173 91) (end 170 88) (width 0.2) (layer "F.Cu") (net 3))
 (segment (start 173 97.96) (end 173 91) (width 0.2) (layer "F.Cu") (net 3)))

